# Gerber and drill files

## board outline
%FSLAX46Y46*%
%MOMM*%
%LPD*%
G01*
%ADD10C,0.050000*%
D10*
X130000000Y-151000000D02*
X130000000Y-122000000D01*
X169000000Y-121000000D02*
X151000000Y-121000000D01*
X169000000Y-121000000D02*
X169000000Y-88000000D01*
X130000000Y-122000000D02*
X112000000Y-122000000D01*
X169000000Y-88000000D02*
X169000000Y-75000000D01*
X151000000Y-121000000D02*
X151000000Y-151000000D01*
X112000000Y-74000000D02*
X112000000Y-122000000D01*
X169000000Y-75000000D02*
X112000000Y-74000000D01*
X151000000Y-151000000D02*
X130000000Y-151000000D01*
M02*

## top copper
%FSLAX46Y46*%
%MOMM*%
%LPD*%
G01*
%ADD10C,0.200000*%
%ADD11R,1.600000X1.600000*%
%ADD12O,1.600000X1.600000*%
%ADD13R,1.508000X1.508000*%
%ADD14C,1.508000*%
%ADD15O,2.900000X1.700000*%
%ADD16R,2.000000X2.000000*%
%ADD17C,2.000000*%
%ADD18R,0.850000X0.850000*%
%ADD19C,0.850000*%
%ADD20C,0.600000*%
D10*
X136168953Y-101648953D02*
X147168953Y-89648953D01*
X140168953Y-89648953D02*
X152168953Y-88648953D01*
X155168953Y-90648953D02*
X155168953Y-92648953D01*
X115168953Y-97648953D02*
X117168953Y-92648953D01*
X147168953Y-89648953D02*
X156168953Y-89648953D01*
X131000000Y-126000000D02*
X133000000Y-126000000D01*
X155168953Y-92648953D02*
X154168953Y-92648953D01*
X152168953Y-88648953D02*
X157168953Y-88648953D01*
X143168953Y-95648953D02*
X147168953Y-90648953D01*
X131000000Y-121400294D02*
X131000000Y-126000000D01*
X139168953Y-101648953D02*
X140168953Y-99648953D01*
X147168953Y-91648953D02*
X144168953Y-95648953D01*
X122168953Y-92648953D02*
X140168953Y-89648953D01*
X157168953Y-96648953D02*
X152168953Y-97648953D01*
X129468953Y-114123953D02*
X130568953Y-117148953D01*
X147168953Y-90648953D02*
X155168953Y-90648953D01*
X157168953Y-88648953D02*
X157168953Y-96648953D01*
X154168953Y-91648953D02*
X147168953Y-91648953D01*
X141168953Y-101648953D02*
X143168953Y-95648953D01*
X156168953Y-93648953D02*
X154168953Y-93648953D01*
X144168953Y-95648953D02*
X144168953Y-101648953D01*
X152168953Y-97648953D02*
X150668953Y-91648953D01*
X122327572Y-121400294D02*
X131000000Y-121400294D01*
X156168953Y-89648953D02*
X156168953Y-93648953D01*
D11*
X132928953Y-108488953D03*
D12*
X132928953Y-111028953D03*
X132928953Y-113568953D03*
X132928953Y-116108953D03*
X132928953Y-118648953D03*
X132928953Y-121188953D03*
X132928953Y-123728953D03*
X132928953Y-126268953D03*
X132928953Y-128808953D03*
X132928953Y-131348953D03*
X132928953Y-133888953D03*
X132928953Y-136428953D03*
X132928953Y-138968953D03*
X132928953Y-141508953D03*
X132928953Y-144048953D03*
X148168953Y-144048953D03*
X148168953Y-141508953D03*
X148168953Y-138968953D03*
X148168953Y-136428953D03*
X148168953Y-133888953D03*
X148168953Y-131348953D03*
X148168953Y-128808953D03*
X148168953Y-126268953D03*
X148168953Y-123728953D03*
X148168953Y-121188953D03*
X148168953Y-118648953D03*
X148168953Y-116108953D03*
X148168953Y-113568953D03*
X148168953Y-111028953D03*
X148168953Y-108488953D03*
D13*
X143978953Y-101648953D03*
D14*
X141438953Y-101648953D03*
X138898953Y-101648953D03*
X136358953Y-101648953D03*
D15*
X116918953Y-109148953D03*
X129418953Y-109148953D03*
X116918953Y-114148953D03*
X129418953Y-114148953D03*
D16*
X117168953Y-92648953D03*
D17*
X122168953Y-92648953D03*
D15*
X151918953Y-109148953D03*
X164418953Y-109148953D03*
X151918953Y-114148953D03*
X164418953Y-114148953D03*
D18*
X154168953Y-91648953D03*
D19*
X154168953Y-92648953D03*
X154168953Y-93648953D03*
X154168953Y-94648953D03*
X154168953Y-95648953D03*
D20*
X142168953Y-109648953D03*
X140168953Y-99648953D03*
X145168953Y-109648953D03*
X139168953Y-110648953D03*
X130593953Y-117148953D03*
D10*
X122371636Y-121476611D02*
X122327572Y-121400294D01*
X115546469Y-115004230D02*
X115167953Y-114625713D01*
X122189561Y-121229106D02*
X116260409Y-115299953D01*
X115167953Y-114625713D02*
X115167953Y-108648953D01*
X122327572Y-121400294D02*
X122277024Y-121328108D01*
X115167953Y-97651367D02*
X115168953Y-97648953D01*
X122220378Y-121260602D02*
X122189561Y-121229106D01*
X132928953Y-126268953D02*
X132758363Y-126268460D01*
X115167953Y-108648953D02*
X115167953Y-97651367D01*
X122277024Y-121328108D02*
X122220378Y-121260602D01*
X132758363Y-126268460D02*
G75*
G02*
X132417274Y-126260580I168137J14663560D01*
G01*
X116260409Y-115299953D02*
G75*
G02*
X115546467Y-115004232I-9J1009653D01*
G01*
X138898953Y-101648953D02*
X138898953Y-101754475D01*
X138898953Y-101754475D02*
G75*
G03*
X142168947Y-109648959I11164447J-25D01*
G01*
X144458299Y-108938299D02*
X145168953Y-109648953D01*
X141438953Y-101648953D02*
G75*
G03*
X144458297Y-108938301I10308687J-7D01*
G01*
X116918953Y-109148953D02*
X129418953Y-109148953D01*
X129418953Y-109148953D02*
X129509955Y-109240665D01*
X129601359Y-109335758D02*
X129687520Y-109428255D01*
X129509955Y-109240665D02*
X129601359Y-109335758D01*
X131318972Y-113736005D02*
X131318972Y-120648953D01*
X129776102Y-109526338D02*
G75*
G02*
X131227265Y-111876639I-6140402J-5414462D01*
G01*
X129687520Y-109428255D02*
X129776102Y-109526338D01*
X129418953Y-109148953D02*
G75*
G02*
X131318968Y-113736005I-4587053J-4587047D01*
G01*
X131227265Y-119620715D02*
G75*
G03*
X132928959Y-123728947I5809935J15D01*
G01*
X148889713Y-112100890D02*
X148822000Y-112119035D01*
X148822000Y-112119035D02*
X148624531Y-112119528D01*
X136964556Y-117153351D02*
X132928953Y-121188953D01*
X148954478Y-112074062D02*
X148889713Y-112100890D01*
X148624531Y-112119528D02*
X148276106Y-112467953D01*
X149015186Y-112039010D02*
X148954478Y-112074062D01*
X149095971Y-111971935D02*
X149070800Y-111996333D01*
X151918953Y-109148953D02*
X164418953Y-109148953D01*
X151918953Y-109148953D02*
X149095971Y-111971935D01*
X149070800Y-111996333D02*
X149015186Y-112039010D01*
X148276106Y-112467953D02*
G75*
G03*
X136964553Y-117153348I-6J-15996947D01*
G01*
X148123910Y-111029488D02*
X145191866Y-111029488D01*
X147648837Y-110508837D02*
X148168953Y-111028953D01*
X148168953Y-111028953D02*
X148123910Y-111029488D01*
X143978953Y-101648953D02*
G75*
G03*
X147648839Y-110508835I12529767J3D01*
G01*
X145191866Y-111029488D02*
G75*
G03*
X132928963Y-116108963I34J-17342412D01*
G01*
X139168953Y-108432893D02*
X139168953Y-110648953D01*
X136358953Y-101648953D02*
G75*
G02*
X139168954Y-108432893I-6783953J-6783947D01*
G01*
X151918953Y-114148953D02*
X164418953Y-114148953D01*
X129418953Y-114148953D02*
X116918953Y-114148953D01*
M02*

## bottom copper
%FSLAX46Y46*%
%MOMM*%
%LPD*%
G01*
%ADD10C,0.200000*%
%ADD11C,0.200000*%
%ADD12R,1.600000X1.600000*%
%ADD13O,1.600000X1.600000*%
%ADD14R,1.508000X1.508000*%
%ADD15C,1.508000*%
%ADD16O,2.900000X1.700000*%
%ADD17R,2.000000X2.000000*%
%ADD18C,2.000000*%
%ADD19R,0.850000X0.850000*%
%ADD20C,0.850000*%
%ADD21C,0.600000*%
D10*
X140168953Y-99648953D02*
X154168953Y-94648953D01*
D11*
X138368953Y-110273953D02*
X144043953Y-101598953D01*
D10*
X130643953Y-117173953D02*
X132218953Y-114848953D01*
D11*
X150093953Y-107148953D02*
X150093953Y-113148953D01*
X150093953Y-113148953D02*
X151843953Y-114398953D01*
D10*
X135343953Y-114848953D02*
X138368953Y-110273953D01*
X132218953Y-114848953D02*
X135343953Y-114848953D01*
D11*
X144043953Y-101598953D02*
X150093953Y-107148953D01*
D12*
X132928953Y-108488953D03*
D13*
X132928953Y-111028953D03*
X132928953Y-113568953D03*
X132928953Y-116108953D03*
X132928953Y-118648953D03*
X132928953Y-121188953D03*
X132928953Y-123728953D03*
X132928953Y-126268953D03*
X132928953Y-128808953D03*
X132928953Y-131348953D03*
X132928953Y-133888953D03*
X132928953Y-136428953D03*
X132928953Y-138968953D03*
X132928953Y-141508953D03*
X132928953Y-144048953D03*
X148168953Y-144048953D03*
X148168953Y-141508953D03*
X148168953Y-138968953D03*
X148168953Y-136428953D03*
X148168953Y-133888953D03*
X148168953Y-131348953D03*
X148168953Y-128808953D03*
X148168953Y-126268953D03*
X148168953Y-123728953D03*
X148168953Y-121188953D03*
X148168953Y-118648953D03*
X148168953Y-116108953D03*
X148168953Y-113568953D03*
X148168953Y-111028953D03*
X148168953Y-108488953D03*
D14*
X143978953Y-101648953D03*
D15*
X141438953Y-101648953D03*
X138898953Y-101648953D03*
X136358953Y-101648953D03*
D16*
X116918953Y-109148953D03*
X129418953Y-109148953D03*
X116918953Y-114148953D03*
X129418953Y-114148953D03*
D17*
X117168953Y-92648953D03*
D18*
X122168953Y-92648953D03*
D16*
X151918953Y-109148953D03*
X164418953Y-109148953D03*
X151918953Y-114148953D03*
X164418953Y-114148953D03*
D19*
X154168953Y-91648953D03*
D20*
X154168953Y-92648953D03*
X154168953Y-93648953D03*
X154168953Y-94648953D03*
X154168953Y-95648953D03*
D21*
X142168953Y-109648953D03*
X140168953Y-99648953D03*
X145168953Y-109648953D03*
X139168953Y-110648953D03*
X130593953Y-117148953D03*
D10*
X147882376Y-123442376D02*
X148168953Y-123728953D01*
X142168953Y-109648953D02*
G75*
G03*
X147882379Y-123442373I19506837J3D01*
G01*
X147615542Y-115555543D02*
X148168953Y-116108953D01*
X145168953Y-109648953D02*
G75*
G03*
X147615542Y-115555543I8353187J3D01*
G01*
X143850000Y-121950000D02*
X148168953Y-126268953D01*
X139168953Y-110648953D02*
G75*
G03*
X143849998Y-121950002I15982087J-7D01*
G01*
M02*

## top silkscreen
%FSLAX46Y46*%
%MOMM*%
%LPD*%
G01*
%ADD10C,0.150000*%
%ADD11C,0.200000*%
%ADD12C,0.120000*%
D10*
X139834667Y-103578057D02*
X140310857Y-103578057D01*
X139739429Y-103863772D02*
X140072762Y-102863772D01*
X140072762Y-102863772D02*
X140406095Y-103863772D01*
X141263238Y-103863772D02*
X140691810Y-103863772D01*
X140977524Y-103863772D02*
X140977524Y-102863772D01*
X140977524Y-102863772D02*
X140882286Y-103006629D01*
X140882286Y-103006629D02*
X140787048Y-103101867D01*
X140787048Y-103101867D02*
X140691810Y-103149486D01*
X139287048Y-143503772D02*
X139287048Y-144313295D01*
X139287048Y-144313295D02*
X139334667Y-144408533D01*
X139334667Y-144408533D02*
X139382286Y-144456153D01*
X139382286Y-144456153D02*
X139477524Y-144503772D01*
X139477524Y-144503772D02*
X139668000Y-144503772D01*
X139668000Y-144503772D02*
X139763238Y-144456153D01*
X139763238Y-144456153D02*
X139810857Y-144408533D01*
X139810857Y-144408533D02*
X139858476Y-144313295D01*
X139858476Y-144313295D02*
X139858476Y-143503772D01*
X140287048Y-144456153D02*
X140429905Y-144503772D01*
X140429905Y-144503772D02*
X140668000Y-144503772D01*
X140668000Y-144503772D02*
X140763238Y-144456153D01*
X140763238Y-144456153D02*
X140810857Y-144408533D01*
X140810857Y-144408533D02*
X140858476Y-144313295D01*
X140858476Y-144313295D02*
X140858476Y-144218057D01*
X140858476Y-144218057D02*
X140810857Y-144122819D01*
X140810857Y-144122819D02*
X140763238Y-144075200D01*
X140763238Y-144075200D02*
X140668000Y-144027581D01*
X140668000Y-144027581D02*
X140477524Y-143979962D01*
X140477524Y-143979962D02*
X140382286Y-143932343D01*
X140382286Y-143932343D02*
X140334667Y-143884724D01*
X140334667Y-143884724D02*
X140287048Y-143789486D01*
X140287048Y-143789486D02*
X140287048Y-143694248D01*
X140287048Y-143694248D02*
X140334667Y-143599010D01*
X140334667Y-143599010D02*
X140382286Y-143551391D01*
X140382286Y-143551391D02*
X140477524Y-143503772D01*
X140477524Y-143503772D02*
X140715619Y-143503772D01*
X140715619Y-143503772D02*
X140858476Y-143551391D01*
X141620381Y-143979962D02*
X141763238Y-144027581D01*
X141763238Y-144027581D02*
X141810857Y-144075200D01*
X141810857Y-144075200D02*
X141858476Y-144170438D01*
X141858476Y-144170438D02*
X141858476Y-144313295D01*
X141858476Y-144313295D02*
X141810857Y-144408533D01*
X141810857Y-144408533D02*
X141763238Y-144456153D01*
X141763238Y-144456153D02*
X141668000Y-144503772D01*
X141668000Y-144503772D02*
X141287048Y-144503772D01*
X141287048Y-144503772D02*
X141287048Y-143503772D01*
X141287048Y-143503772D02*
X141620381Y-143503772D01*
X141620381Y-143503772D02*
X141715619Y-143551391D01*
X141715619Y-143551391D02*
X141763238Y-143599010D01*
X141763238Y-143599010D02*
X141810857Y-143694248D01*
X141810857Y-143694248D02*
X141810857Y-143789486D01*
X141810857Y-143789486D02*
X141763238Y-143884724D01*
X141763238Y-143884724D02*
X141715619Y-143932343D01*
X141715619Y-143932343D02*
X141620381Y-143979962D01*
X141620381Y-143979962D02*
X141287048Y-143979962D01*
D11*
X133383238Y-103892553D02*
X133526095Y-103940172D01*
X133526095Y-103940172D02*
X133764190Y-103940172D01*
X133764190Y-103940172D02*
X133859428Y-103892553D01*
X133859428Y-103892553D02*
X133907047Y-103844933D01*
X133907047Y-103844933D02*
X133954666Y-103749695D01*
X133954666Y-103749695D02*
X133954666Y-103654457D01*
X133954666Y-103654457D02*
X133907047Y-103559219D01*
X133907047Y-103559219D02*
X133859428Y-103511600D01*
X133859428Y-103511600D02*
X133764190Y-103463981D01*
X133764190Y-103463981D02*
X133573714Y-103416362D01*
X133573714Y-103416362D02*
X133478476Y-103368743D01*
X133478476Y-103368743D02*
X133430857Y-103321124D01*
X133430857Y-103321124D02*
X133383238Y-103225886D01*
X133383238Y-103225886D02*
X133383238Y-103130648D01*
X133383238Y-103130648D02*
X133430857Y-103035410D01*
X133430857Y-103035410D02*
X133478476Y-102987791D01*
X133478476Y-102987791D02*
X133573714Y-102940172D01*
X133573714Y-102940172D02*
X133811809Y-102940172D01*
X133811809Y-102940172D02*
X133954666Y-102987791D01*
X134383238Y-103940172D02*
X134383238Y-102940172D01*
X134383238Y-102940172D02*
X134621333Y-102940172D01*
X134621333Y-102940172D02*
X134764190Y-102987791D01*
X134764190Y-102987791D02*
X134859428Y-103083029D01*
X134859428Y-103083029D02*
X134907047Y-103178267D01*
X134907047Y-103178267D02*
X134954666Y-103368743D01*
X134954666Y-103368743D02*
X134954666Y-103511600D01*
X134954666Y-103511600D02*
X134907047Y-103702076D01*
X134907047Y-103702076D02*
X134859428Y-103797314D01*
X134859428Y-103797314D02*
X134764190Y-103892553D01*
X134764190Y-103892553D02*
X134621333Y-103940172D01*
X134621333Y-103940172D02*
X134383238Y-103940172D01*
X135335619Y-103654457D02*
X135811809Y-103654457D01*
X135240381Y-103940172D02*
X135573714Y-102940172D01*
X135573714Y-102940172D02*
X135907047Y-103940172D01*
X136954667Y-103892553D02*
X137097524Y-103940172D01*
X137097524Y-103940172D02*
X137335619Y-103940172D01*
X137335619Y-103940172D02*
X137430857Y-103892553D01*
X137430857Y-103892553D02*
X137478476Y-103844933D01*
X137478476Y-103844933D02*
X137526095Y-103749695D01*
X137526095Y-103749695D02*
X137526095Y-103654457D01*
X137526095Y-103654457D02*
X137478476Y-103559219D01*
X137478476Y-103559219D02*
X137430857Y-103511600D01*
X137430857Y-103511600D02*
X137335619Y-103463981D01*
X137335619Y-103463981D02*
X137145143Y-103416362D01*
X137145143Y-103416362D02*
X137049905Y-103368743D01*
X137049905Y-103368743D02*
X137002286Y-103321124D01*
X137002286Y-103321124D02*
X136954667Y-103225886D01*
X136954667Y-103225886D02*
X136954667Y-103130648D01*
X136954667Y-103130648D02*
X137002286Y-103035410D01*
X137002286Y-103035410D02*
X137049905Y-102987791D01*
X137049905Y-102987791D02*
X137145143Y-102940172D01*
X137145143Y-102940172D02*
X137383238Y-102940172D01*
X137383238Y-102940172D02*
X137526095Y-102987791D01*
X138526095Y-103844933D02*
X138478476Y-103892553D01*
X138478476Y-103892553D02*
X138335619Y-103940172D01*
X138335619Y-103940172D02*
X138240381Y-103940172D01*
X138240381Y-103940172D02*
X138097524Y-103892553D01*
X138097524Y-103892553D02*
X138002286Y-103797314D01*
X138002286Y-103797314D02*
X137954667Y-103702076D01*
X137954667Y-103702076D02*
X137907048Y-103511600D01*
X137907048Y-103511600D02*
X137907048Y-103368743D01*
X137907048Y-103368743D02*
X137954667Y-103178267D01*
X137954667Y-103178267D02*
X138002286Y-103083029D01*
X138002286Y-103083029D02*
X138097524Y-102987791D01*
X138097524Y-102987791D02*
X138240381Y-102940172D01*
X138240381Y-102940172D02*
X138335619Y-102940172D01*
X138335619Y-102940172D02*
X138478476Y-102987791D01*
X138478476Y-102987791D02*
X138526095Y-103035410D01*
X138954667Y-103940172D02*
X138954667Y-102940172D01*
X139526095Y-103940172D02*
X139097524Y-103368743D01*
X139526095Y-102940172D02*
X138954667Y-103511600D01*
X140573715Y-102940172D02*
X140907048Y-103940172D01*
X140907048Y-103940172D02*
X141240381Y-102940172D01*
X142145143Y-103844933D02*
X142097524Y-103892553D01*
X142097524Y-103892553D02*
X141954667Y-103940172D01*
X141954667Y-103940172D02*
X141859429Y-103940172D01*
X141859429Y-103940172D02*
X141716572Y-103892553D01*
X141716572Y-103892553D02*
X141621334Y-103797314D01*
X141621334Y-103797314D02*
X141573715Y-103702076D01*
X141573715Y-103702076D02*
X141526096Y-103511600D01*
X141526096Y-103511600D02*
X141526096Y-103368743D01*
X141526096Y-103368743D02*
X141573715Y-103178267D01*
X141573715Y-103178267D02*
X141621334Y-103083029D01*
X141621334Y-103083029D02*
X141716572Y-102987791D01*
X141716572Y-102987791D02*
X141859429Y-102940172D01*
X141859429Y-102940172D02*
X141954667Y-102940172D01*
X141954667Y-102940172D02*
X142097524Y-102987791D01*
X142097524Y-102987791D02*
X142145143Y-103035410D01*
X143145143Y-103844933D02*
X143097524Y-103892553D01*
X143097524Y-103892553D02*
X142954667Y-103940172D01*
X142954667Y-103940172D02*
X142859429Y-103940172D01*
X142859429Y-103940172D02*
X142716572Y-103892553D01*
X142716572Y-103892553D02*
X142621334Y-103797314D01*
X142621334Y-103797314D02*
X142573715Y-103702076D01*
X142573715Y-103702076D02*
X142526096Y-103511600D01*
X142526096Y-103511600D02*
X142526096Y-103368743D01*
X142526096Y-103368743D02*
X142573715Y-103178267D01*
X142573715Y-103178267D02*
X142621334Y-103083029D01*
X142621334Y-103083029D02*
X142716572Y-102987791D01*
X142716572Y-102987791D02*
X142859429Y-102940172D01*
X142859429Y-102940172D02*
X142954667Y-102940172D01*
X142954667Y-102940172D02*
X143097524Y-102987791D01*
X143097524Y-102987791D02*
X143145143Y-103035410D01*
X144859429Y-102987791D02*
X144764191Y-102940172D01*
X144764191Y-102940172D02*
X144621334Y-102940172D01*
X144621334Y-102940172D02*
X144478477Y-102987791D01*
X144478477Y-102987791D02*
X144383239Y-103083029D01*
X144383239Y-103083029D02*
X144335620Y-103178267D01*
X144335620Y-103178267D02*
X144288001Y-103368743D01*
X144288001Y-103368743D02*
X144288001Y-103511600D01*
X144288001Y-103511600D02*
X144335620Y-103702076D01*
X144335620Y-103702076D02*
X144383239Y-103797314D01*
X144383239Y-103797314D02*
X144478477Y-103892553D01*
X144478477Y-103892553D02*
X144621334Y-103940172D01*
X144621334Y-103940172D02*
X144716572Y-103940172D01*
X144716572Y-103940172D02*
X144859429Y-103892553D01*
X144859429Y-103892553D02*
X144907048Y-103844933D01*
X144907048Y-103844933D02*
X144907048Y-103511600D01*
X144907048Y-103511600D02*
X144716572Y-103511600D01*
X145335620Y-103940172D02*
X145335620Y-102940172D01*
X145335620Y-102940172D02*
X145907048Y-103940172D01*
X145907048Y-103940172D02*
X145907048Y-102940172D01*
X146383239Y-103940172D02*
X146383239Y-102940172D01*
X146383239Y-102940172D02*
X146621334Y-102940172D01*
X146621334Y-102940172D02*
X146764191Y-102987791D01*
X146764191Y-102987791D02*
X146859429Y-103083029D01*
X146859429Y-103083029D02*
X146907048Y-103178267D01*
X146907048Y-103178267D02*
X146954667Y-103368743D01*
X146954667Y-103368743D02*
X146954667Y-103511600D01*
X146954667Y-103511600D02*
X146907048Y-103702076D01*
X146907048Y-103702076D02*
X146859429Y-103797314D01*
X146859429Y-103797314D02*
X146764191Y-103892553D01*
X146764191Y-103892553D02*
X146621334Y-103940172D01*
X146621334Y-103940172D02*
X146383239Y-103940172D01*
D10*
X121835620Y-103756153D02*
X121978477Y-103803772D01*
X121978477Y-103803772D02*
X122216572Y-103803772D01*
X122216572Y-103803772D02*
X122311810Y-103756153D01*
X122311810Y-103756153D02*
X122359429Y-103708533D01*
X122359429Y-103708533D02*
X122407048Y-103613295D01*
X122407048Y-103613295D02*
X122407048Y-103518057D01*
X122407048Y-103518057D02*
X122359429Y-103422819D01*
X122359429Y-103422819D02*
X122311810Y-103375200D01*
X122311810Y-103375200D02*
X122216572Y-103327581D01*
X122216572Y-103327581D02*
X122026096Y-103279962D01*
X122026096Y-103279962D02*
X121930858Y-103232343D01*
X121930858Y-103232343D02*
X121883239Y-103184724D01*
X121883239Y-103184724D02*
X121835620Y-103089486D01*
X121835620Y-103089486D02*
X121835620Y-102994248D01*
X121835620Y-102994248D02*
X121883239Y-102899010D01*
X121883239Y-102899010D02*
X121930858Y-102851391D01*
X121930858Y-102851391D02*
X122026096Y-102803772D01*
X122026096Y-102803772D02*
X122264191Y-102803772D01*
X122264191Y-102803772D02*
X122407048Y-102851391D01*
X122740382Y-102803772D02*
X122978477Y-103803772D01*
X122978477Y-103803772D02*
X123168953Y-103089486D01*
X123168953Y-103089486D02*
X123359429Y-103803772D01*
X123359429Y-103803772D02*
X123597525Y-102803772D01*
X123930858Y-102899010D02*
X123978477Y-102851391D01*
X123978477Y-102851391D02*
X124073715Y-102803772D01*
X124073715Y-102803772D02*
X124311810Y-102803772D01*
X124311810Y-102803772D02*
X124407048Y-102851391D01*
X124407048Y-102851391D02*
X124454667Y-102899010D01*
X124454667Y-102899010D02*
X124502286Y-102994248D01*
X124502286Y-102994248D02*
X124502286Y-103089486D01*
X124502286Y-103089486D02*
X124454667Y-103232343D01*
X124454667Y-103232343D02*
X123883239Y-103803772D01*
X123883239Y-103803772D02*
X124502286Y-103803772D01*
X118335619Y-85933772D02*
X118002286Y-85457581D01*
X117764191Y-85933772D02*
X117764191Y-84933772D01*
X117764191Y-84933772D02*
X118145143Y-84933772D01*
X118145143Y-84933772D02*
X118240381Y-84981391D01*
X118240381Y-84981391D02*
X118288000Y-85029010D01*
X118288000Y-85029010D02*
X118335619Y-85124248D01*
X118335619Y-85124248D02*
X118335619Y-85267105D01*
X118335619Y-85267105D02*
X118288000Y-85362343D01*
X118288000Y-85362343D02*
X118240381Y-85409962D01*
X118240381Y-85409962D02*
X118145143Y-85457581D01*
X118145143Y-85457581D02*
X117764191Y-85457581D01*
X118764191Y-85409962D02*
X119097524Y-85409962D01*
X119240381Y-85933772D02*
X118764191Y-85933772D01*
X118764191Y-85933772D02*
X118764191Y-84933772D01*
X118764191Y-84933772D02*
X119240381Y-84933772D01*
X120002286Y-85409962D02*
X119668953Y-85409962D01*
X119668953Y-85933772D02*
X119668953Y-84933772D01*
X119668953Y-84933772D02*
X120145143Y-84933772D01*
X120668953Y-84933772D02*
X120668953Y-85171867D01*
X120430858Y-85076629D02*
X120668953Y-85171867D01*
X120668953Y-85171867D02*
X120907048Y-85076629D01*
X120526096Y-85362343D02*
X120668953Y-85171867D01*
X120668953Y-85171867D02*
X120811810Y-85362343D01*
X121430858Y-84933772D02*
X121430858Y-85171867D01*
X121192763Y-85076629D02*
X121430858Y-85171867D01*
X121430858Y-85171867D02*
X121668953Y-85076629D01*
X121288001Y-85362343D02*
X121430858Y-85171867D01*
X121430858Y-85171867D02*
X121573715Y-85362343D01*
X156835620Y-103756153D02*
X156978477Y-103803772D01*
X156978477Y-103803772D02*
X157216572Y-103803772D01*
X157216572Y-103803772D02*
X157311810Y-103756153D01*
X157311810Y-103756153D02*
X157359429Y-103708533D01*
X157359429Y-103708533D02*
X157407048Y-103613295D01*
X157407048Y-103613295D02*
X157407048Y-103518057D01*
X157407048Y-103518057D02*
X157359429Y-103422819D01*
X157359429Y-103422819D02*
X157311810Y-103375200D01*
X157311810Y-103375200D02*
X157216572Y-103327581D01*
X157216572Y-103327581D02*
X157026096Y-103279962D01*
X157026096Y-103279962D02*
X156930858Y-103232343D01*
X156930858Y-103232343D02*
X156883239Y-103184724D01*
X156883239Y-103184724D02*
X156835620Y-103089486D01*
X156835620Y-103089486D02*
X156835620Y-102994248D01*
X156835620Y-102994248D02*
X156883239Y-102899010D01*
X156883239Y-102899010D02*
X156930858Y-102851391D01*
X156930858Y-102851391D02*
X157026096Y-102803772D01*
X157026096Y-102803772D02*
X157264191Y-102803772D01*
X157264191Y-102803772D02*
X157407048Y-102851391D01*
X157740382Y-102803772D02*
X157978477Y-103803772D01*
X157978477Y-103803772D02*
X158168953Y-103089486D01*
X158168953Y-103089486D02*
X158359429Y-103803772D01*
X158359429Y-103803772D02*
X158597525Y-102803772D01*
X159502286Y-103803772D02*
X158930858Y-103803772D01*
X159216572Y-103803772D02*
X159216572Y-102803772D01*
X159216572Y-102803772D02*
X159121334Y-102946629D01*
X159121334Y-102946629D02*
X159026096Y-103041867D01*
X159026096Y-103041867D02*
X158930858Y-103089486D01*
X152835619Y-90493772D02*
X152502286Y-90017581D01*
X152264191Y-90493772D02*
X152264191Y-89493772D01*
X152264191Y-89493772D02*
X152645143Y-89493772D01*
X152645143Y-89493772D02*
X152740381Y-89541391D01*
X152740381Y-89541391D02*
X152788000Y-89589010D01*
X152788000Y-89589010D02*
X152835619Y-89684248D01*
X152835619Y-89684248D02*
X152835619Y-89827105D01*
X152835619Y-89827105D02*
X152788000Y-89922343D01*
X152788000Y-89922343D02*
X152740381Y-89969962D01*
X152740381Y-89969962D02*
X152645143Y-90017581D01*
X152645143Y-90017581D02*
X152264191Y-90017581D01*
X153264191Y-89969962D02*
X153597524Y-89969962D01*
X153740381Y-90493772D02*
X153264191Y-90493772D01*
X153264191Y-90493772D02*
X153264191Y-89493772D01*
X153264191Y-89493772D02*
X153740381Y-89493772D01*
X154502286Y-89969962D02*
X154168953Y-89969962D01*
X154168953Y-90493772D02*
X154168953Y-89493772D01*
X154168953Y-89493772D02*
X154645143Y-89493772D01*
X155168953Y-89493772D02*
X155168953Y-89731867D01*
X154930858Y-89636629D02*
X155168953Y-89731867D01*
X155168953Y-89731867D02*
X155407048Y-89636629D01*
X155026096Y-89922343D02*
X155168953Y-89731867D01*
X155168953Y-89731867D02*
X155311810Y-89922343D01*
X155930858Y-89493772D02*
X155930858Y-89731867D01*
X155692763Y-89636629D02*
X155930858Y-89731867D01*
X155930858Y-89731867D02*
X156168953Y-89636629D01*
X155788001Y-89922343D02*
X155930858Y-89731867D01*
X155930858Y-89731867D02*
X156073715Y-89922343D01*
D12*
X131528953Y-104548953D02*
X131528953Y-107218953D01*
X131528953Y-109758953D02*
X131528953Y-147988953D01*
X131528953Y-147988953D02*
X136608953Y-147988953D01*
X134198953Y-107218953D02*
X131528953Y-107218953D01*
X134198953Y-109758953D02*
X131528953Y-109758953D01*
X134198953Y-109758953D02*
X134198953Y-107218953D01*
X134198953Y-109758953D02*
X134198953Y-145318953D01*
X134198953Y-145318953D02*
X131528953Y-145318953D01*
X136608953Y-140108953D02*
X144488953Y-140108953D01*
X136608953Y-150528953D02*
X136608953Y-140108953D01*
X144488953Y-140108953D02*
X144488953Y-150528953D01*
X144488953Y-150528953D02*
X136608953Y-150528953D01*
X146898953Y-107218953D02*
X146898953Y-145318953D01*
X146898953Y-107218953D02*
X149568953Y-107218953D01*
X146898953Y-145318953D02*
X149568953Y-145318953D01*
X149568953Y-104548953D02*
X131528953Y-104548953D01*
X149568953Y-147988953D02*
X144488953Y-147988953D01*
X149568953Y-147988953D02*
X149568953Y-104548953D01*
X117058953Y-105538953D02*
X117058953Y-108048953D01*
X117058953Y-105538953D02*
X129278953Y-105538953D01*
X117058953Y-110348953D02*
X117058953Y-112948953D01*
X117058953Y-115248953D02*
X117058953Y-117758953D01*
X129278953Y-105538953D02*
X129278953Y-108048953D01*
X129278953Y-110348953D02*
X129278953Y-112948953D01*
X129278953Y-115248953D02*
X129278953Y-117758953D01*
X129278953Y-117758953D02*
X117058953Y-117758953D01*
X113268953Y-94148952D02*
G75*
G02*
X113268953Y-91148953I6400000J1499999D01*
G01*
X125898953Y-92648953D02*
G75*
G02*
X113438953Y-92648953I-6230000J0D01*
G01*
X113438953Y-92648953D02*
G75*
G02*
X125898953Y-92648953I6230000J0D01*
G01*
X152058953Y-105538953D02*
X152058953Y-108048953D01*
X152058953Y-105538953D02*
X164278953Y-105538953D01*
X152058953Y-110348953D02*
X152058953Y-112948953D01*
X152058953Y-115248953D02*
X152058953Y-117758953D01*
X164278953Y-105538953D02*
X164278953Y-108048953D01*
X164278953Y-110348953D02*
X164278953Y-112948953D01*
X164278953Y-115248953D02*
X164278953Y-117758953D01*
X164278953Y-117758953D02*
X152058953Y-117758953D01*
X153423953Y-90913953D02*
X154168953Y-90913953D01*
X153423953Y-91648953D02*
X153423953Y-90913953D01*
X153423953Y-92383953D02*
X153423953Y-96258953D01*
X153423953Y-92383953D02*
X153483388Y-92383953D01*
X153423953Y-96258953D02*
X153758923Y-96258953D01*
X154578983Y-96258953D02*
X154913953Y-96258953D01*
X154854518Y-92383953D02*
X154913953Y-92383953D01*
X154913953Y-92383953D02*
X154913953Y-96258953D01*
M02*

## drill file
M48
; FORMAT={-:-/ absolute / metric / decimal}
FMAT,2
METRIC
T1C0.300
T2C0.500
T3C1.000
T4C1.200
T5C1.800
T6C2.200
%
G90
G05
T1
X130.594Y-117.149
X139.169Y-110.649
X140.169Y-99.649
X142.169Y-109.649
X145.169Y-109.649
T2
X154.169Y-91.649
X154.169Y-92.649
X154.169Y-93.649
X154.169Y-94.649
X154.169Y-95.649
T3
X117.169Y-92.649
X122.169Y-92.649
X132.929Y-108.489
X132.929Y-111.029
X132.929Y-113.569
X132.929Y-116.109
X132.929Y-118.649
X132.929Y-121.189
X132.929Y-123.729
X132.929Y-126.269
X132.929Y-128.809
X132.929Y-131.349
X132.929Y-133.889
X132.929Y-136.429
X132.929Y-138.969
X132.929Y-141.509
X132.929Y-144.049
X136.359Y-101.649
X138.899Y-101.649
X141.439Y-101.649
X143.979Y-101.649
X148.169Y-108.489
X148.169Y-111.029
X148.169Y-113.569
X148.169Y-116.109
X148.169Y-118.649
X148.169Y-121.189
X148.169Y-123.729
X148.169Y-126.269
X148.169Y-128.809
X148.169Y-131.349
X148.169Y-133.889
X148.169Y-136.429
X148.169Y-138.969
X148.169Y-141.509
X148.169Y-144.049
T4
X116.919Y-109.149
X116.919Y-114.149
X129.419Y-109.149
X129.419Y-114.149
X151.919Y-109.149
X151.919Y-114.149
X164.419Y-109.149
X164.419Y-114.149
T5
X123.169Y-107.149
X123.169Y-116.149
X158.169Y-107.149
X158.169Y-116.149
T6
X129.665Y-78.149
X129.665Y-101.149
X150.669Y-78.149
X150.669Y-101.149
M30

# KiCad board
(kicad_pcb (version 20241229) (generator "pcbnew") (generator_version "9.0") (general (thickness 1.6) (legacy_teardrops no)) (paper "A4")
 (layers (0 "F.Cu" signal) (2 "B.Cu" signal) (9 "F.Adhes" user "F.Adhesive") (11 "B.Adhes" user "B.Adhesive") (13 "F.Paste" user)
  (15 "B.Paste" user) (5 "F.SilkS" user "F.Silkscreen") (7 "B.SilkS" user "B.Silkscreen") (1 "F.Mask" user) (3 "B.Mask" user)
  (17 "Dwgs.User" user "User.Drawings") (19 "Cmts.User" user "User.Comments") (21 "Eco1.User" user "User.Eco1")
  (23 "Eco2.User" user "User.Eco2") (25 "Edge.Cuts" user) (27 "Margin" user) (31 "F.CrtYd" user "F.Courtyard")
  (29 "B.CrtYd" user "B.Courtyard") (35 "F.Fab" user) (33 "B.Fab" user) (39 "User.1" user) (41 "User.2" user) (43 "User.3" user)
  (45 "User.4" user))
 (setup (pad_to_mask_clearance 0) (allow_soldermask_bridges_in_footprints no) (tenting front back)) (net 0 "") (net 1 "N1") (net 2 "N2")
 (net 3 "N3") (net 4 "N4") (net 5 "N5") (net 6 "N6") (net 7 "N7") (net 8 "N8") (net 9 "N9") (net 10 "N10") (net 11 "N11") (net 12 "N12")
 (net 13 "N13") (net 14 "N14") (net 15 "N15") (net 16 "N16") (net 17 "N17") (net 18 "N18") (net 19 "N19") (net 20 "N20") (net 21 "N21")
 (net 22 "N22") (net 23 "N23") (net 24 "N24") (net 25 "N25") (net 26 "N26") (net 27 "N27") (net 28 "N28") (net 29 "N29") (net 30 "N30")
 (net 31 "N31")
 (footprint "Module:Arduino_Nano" (layer "F.Cu") (at 132.928953 108.488953)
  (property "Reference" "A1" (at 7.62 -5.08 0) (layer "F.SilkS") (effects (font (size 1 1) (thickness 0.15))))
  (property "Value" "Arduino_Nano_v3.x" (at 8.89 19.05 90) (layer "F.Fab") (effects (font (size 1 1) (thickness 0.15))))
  (fp_line (start -1.4 -3.94) (end -1.4 -1.27) (stroke (width 0.12) (type solid)) (layer "F.SilkS"))
  (fp_line (start -1.4 1.27) (end -1.4 39.5) (stroke (width 0.12) (type solid)) (layer "F.SilkS"))
  (fp_line (start -1.4 39.5) (end 3.68 39.5) (stroke (width 0.12) (type solid)) (layer "F.SilkS"))
  (fp_line (start 1.27 -1.27) (end -1.4 -1.27) (stroke (width 0.12) (type solid)) (layer "F.SilkS"))
  (fp_line (start 1.27 1.27) (end -1.4 1.27) (stroke (width 0.12) (type solid)) (layer "F.SilkS"))
  (fp_line (start 1.27 1.27) (end 1.27 -1.27) (stroke (width 0.12) (type solid)) (layer "F.SilkS"))
  (fp_line (start 1.27 1.27) (end 1.27 36.83) (stroke (width 0.12) (type solid)) (layer "F.SilkS"))
  (fp_line (start 1.27 36.83) (end -1.4 36.83) (stroke (width 0.12) (type solid)) (layer "F.SilkS"))
  (fp_line (start 3.68 31.62) (end 11.56 31.62) (stroke (width 0.12) (type solid)) (layer "F.SilkS"))
  (fp_line (start 3.68 42.04) (end 3.68 31.62) (stroke (width 0.12) (type solid)) (layer "F.SilkS"))
  (fp_line (start 11.56 31.62) (end 11.56 42.04) (stroke (width 0.12) (type solid)) (layer "F.SilkS"))
  (fp_line (start 11.56 42.04) (end 3.68 42.04) (stroke (width 0.12) (type solid)) (layer "F.SilkS"))
  (fp_line (start 13.97 -1.27) (end 13.97 36.83) (stroke (width 0.12) (type solid)) (layer "F.SilkS"))
  (fp_line (start 13.97 -1.27) (end 16.64 -1.27) (stroke (width 0.12) (type solid)) (layer "F.SilkS"))
  (fp_line (start 13.97 36.83) (end 16.64 36.83) (stroke (width 0.12) (type solid)) (layer "F.SilkS"))
  (fp_line (start 16.64 -3.94) (end -1.4 -3.94) (stroke (width 0.12) (type solid)) (layer "F.SilkS"))
  (fp_line (start 16.64 39.5) (end 11.56 39.5) (stroke (width 0.12) (type solid)) (layer "F.SilkS"))
  (fp_line (start 16.64 39.5) (end 16.64 -3.94) (stroke (width 0.12) (type solid)) (layer "F.SilkS"))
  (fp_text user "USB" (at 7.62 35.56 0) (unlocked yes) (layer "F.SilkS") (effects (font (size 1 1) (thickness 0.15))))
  (pad "1" thru_hole rect (at 0 0) (size 1.6 1.6) (drill 1) (layers "*.Cu" "*.Mask") (remove_unused_layers no) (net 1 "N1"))
  (pad "2" thru_hole oval (at 0 2.54) (size 1.6 1.6) (drill 1) (layers "*.Cu" "*.Mask") (remove_unused_layers no) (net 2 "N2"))
  (pad "3" thru_hole oval (at 0 5.08) (size 1.6 1.6) (drill 1) (layers "*.Cu" "*.Mask") (remove_unused_layers no) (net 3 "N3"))
  (pad "4" thru_hole oval (at 0 7.62) (size 1.6 1.6) (drill 1) (layers "*.Cu" "*.Mask") (remove_unused_layers no) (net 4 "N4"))
  (pad "5" thru_hole oval (at 0 10.16) (size 1.6 1.6) (drill 1) (layers "*.Cu" "*.Mask") (remove_unused_layers no) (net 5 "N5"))
  (pad "6" thru_hole oval (at 0 12.7) (size 1.6 1.6) (drill 1) (layers "*.Cu" "*.Mask") (remove_unused_layers no) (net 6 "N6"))
  (pad "7" thru_hole oval (at 0 15.24) (size 1.6 1.6) (drill 1) (layers "*.Cu" "*.Mask") (remove_unused_layers no) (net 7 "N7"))
  (pad "8" thru_hole oval (at 0 17.78) (size 1.6 1.6) (drill 1) (layers "*.Cu" "*.Mask") (remove_unused_layers no) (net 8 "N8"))
  (pad "9" thru_hole oval (at 0 20.32) (size 1.6 1.6) (drill 1) (layers "*.Cu" "*.Mask") (remove_unused_layers no) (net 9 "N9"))
  (pad "10" thru_hole oval (at 0 22.86) (size 1.6 1.6) (drill 1) (layers "*.Cu" "*.Mask") (remove_unused_layers no) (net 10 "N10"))
  (pad "11" thru_hole oval (at 0 25.4) (size 1.6 1.6) (drill 1) (layers "*.Cu" "*.Mask") (remove_unused_layers no) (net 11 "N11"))
  (pad "12" thru_hole oval (at 0 27.94) (size 1.6 1.6) (drill 1) (layers "*.Cu" "*.Mask") (remove_unused_layers no) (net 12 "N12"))
  (pad "13" thru_hole oval (at 0 30.48) (size 1.6 1.6) (drill 1) (layers "*.Cu" "*.Mask") (remove_unused_layers no) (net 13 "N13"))
  (pad "14" thru_hole oval (at 0 33.02) (size 1.6 1.6) (drill 1) (layers "*.Cu" "*.Mask") (remove_unused_layers no) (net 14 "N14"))
  (pad "15" thru_hole oval (at 0 35.56) (size 1.6 1.6) (drill 1) (layers "*.Cu" "*.Mask") (remove_unused_layers no) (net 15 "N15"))
  (pad "16" thru_hole oval (at 15.24 35.56) (size 1.6 1.6) (drill 1) (layers "*.Cu" "*.Mask") (remove_unused_layers no) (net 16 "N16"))
  (pad "17" thru_hole oval (at 15.24 33.02) (size 1.6 1.6) (drill 1) (layers "*.Cu" "*.Mask") (remove_unused_layers no) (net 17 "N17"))
  (pad "18" thru_hole oval (at 15.24 30.48) (size 1.6 1.6) (drill 1) (layers "*.Cu" "*.Mask") (remove_unused_layers no) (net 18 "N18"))
  (pad "19" thru_hole oval (at 15.24 27.94) (size 1.6 1.6) (drill 1) (layers "*.Cu" "*.Mask") (remove_unused_layers no) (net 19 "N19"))
  (pad "20" thru_hole oval (at 15.24 25.4) (size 1.6 1.6) (drill 1) (layers "*.Cu" "*.Mask") (remove_unused_layers no) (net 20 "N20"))
  (pad "21" thru_hole oval (at 15.24 22.86) (size 1.6 1.6) (drill 1) (layers "*.Cu" "*.Mask") (remove_unused_layers no) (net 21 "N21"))
  (pad "22" thru_hole oval (at 15.24 20.32) (size 1.6 1.6) (drill 1) (layers "*.Cu" "*.Mask") (remove_unused_layers no) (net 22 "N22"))
  (pad "23" thru_hole oval (at 15.24 17.78) (size 1.6 1.6) (drill 1) (layers "*.Cu" "*.Mask") (remove_unused_layers no) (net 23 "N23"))
  (pad "24" thru_hole oval (at 15.24 15.24) (size 1.6 1.6) (drill 1) (layers "*.Cu" "*.Mask") (remove_unused_layers no) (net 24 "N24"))
  (pad "25" thru_hole oval (at 15.24 12.7) (size 1.6 1.6) (drill 1) (layers "*.Cu" "*.Mask") (remove_unused_layers no) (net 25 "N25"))
  (pad "26" thru_hole oval (at 15.24 10.16) (size 1.6 1.6) (drill 1) (layers "*.Cu" "*.Mask") (remove_unused_layers no) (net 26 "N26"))
  (pad "27" thru_hole oval (at 15.24 7.62) (size 1.6 1.6) (drill 1) (layers "*.Cu" "*.Mask") (remove_unused_layers no) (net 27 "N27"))
  (pad "28" thru_hole oval (at 15.24 5.08) (size 1.6 1.6) (drill 1) (layers "*.Cu" "*.Mask") (remove_unused_layers no) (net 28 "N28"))
  (pad "29" thru_hole oval (at 15.24 2.54) (size 1.6 1.6) (drill 1) (layers "*.Cu" "*.Mask") (remove_unused_layers no) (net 4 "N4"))
  (pad "30" thru_hole oval (at 15.24 0) (size 1.6 1.6) (drill 1) (layers "*.Cu" "*.Mask") (remove_unused_layers no) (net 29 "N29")))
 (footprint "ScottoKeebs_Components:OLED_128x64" (layer "F.Cu") (at 140.168953 89.648953)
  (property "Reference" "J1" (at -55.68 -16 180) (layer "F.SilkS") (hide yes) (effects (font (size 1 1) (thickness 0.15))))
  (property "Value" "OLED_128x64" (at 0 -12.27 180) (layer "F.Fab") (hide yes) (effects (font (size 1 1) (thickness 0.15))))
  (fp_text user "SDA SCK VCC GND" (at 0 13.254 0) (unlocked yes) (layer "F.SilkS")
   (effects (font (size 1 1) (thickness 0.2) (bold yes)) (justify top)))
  (pad "" np_thru_hole circle (at -10.50445 -11.5 180) (size 2.2 2.2) (drill 2.2) (layers "*.Cu" "*.Mask") (solder_mask_margin 0.102))
  (pad "" np_thru_hole circle (at -10.50445 11.5 180) (size 2.2 2.2) (drill 2.2) (layers "*.Cu" "*.Mask") (solder_mask_margin 0.102))
  (pad "" np_thru_hole circle (at 10.5 -11.5 180) (size 2.2 2.2) (drill 2.2) (layers "*.Cu" "*.Mask") (solder_mask_margin 0.102))
  (pad "" np_thru_hole circle (at 10.5 11.5 180) (size 2.2 2.2) (drill 2.2) (layers "*.Cu" "*.Mask") (solder_mask_margin 0.102))
  (pad "1" thru_hole rect (at 3.81 12 180) (size 1.508 1.508) (drill 1) (layers "*.Cu" "*.Mask") (remove_unused_layers no) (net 4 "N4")
   (solder_mask_margin 0.102))
  (pad "2" thru_hole circle (at 1.27 12 180) (size 1.508 1.508) (drill 1) (layers "*.Cu" "*.Mask") (remove_unused_layers no) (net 27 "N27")
   (solder_mask_margin 0.102))
  (pad "3" thru_hole circle (at -1.27 12 180) (size 1.508 1.508) (drill 1) (layers "*.Cu" "*.Mask") (remove_unused_layers no) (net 24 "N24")
   (solder_mask_margin 0.102))
  (pad "4" thru_hole circle (at -3.81 12 180) (size 1.508 1.508) (drill 1) (layers "*.Cu" "*.Mask") (remove_unused_layers no) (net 23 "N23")
   (solder_mask_margin 0.102)))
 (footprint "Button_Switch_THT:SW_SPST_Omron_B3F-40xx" (layer "F.Cu") (at 116.918953 109.148953)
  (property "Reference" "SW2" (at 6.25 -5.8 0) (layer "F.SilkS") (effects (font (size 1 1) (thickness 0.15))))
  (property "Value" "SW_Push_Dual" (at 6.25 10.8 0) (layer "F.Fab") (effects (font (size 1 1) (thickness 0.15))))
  (fp_line (start 0.14 -3.61) (end 0.14 -1.1) (stroke (width 0.12) (type default)) (layer "F.SilkS"))
  (fp_line (start 0.14 -3.61) (end 12.36 -3.61) (stroke (width 0.12) (type default)) (layer "F.SilkS"))
  (fp_line (start 0.14 1.2) (end 0.14 3.8) (stroke (width 0.12) (type default)) (layer "F.SilkS"))
  (fp_line (start 0.14 6.1) (end 0.14 8.61) (stroke (width 0.12) (type default)) (layer "F.SilkS"))
  (fp_line (start 12.36 -3.61) (end 12.36 -1.1) (stroke (width 0.12) (type default)) (layer "F.SilkS"))
  (fp_line (start 12.36 1.2) (end 12.36 3.8) (stroke (width 0.12) (type default)) (layer "F.SilkS"))
  (fp_line (start 12.36 6.1) (end 12.36 8.61) (stroke (width 0.12) (type default)) (layer "F.SilkS"))
  (fp_line (start 12.36 8.61) (end 0.14 8.61) (stroke (width 0.12) (type default)) (layer "F.SilkS"))
  (pad "" np_thru_hole circle (at 6.25 -2) (size 1.8 1.8) (drill 1.8) (layers "*.Cu" "*.Mask"))
  (pad "" np_thru_hole circle (at 6.25 7) (size 1.8 1.8) (drill 1.8) (layers "*.Cu" "*.Mask"))
  (pad "1" thru_hole oval (at 0 0) (size 2.9 1.7) (drill 1.2) (layers "*.Cu" "*.Mask") (remove_unused_layers no) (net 7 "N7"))
  (pad "1" thru_hole oval (at 12.5 0) (size 2.9 1.7) (drill 1.2) (layers "*.Cu" "*.Mask") (remove_unused_layers no) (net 7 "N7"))
  (pad "2" thru_hole oval (at 0 5) (size 2.9 1.7) (drill 1.2) (layers "*.Cu" "*.Mask") (remove_unused_layers no) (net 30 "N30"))
  (pad "2" thru_hole oval (at 12.5 5) (size 2.9 1.7) (drill 1.2) (layers "*.Cu" "*.Mask") (remove_unused_layers no) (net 30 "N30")))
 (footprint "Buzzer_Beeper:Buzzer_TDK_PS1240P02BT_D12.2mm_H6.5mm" (layer "F.Cu") (at 117.168953 92.648953)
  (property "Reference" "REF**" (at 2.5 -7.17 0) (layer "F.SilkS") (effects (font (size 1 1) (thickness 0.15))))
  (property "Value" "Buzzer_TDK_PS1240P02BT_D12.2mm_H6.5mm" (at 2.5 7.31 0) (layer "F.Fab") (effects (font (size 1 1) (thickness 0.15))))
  (fp_arc (start -3.9 1.499999) (mid -4.073431 0) (end -3.9 -1.5) (stroke (width 0.12) (type solid)) (layer "F.SilkS"))
  (fp_circle (center 2.5 0) (end 8.73 0) (stroke (width 0.12) (type solid)) (fill no) (layer "F.SilkS"))
  (pad "1" thru_hole rect (at 0 0) (size 2 2) (drill 1) (layers "*.Cu" "*.Mask") (remove_unused_layers no))
  (pad "2" thru_hole circle (at 5 0) (size 2 2) (drill 1) (layers "*.Cu" "*.Mask") (remove_unused_layers no)))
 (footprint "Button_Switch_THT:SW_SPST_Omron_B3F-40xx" (layer "F.Cu") (at 151.918953 109.148953)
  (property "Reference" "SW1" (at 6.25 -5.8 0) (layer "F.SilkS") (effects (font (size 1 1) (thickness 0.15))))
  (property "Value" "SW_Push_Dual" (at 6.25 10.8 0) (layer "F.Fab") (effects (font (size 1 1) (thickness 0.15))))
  (fp_line (start 0.14 -3.61) (end 0.14 -1.1) (stroke (width 0.12) (type default)) (layer "F.SilkS"))
  (fp_line (start 0.14 -3.61) (end 12.36 -3.61) (stroke (width 0.12) (type default)) (layer "F.SilkS"))
  (fp_line (start 0.14 1.2) (end 0.14 3.8) (stroke (width 0.12) (type default)) (layer "F.SilkS"))
  (fp_line (start 0.14 6.1) (end 0.14 8.61) (stroke (width 0.12) (type default)) (layer "F.SilkS"))
  (fp_line (start 12.36 -3.61) (end 12.36 -1.1) (stroke (width 0.12) (type default)) (layer "F.SilkS"))
  (fp_line (start 12.36 1.2) (end 12.36 3.8) (stroke (width 0.12) (type default)) (layer "F.SilkS"))
  (fp_line (start 12.36 6.1) (end 12.36 8.61) (stroke (width 0.12) (type default)) (layer "F.SilkS"))
  (fp_line (start 12.36 8.61) (end 0.14 8.61) (stroke (width 0.12) (type default)) (layer "F.SilkS"))
  (pad "" np_thru_hole circle (at 6.25 -2) (size 1.8 1.8) (drill 1.8) (layers "*.Cu" "*.Mask"))
  (pad "" np_thru_hole circle (at 6.25 7) (size 1.8 1.8) (drill 1.8) (layers "*.Cu" "*.Mask"))
  (pad "1" thru_hole oval (at 0 0) (size 2.9 1.7) (drill 1.2) (layers "*.Cu" "*.Mask") (remove_unused_layers no) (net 6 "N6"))
  (pad "1" thru_hole oval (at 12.5 0) (size 2.9 1.7) (drill 1.2) (layers "*.Cu" "*.Mask") (remove_unused_layers no) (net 6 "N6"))
  (pad "2" thru_hole oval (at 0 5) (size 2.9 1.7) (drill 1.2) (layers "*.Cu" "*.Mask") (remove_unused_layers no) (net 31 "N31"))
  (pad "2" thru_hole oval (at 12.5 5) (size 2.9 1.7) (drill 1.2) (layers "*.Cu" "*.Mask") (remove_unused_layers no) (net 31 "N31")))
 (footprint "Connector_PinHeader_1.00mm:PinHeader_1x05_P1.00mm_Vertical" (layer "F.Cu") (at 154.168953 91.648953)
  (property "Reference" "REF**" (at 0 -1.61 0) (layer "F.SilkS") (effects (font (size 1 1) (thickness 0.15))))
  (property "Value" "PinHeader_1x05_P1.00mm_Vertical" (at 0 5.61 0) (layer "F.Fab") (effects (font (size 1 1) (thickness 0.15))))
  (fp_line (start -0.745 -0.735) (end 0 -0.735) (stroke (width 0.12) (type solid)) (layer "F.SilkS"))
  (fp_line (start -0.745 0) (end -0.745 -0.735) (stroke (width 0.12) (type solid)) (layer "F.SilkS"))
  (fp_line (start -0.745 0.735) (end -0.745 4.61) (stroke (width 0.12) (type solid)) (layer "F.SilkS"))
  (fp_line (start -0.745 0.735) (end -0.685565 0.735) (stroke (width 0.12) (type solid)) (layer "F.SilkS"))
  (fp_line (start -0.745 4.61) (end -0.41003 4.61) (stroke (width 0.12) (type solid)) (layer "F.SilkS"))
  (fp_line (start 0.41003 4.61) (end 0.745 4.61) (stroke (width 0.12) (type solid)) (layer "F.SilkS"))
  (fp_line (start 0.685565 0.735) (end 0.745 0.735) (stroke (width 0.12) (type solid)) (layer "F.SilkS"))
  (fp_line (start 0.745 0.735) (end 0.745 4.61) (stroke (width 0.12) (type solid)) (layer "F.SilkS"))
  (pad "1" thru_hole rect (at 0 0) (size 0.85 0.85) (drill 0.5) (layers "*.Cu" "*.Mask") (remove_unused_layers no))
  (pad "2" thru_hole circle (at 0 1) (size 0.85 0.85) (drill 0.5) (layers "*.Cu" "*.Mask") (remove_unused_layers no))
  (pad "3" thru_hole circle (at 0 2) (size 0.85 0.85) (drill 0.5) (layers "*.Cu" "*.Mask") (remove_unused_layers no))
  (pad "4" thru_hole circle (at 0 3) (size 0.85 0.85) (drill 0.5) (layers "*.Cu" "*.Mask") (remove_unused_layers no))
  (pad "5" thru_hole circle (at 0 4) (size 0.85 0.85) (drill 0.5) (layers "*.Cu" "*.Mask") (remove_unused_layers no)))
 (gr_line (start 136.168953 101.648953) (end 147.168953 89.648953) (stroke (width 0.2) (type default)) (layer "F.Cu") (net 23))
 (gr_line (start 140.168953 89.648953) (end 152.168953 88.648953) (stroke (width 0.2) (type default)) (layer "F.Cu") (net 4))
 (gr_line (start 155.168953 90.648953) (end 155.168953 92.648953) (stroke (width 0.2) (type default)) (layer "F.Cu") (net 27))
 (gr_line (start 115.168953 97.648953) (end 117.168953 92.648953) (stroke (width 0.2) (type default)) (layer "F.Cu") (net 8))
 (gr_line (start 147.168953 89.648953) (end 156.168953 89.648953) (stroke (width 0.2) (type default)) (layer "F.Cu") (net 23))
 (gr_line (start 131 126) (end 133 126) (stroke (width 0.2) (type default)) (layer "F.Cu") (net 8))
 (gr_line (start 155.168953 92.648953) (end 154.168953 92.648953) (stroke (width 0.2) (type default)) (layer "F.Cu") (net 27))
 (gr_line (start 152.168953 88.648953) (end 157.168953 88.648953) (stroke (width 0.2) (type default)) (layer "F.Cu") (net 4))
 (gr_line (start 143.168953 95.648953) (end 147.168953 90.648953) (stroke (width 0.2) (type default)) (layer "F.Cu") (net 27))
 (gr_line (start 131 121.400294) (end 131 126) (stroke (width 0.2) (type default)) (layer "F.Cu") (net 8))
 (gr_line (start 139.168953 101.648953) (end 140.168953 99.648953) (stroke (width 0.2) (type default)) (layer "F.Cu") (net 24))
 (gr_line (start 147.168953 91.648953) (end 144.168953 95.648953) (stroke (width 0.2) (type default)) (layer "F.Cu") (net 4))
 (gr_line (start 122.168953 92.648953) (end 140.168953 89.648953) (stroke (width 0.2) (type default)) (layer "F.Cu") (net 4))
 (gr_line (start 157.168953 96.648953) (end 152.168953 97.648953) (stroke (width 0.2) (type default)) (layer "F.Cu") (net 4))
 (gr_line (start 129.468953 114.123953) (end 130.568953 117.148953) (stroke (width 0.2) (type default)) (layer "F.Cu") (net 30))
 (gr_line (start 147.168953 90.648953) (end 155.168953 90.648953) (stroke (width 0.2) (type default)) (layer "F.Cu") (net 27))
 (gr_line (start 157.168953 88.648953) (end 157.168953 96.648953) (stroke (width 0.2) (type default)) (layer "F.Cu") (net 4))
 (gr_line (start 154.168953 91.648953) (end 147.168953 91.648953) (stroke (width 0.2) (type default)) (layer "F.Cu") (net 4))
 (gr_line (start 141.168953 101.648953) (end 143.168953 95.648953) (stroke (width 0.2) (type default)) (layer "F.Cu") (net 27))
 (gr_line (start 156.168953 93.648953) (end 154.168953 93.648953) (stroke (width 0.2) (type default)) (layer "F.Cu") (net 23))
 (gr_line (start 144.168953 95.648953) (end 144.168953 101.648953) (stroke (width 0.2) (type default)) (layer "F.Cu") (net 4))
 (gr_line (start 152.168953 97.648953) (end 150.668953 91.648953) (stroke (width 0.2) (type default)) (layer "F.Cu") (net 4))
 (gr_line (start 122.327572 121.400294) (end 131 121.400294) (stroke (width 0.2) (type default)) (layer "F.Cu") (net 8))
 (gr_line (start 156.168953 89.648953) (end 156.168953 93.648953) (stroke (width 0.2) (type default)) (layer "F.Cu") (net 23))
 (gr_line (start 140.168953 99.648953) (end 154.168953 94.648953) (stroke (width 0.2) (type default)) (layer "B.Cu") (net 24))
 (gr_line (start 138.368953 110.273953) (end 144.043953 101.598953) (stroke (width 0.2) (type default)) (layer "B.Cu"))
 (gr_line (start 130.643953 117.173953) (end 132.218953 114.848953) (stroke (width 0.2) (type default)) (layer "B.Cu") (net 30))
 (gr_line (start 150.093953 107.148953) (end 150.093953 113.148953) (stroke (width 0.2) (type default)) (layer "B.Cu"))
 (gr_line (start 150.093953 113.148953) (end 151.843953 114.398953) (stroke (width 0.2) (type default)) (layer "B.Cu"))
 (gr_line (start 135.343953 114.848953) (end 138.368953 110.273953) (stroke (width 0.2) (type default)) (layer "B.Cu") (net 30))
 (gr_line (start 132.218953 114.848953) (end 135.343953 114.848953) (stroke (width 0.2) (type default)) (layer "B.Cu") (net 30))
 (gr_line (start 144.043953 101.598953) (end 150.093953 107.148953) (stroke (width 0.2) (type default)) (layer "B.Cu"))
 (gr_line (start 130 151) (end 130 122) (stroke (width 0.05) (type default)) (layer "Edge.Cuts"))
 (gr_line (start 169 121) (end 151 121) (stroke (width 0.05) (type default)) (layer "Edge.Cuts"))
 (gr_line (start 169 121) (end 169 88) (stroke (width 0.05) (type default)) (layer "Edge.Cuts"))
 (gr_line (start 130 122) (end 112 122) (stroke (width 0.05) (type default)) (layer "Edge.Cuts"))
 (gr_line (start 169 88) (end 169 75) (stroke (width 0.05) (type default)) (layer "Edge.Cuts"))
 (gr_line (start 151 121) (end 151 151) (stroke (width 0.05) (type default)) (layer "Edge.Cuts"))
 (gr_line (start 112 74) (end 112 122) (stroke (width 0.05) (type default)) (layer "Edge.Cuts"))
 (gr_line (start 169 75) (end 112 74) (stroke (width 0.05) (type default)) (layer "Edge.Cuts"))
 (gr_line (start 151 151) (end 130 151) (stroke (width 0.05) (type default)) (layer "Edge.Cuts"))
 (segment (start 122.371636 121.476611) (end 122.327572 121.400294) (width 0.2) (layer "F.Cu") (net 8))
 (segment (start 115.546469 115.00423) (end 115.167953 114.625713) (width 0.2) (layer "F.Cu") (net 8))
 (segment (start 122.189561 121.229106) (end 116.260409 115.299953) (width 0.2) (layer "F.Cu") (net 8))
 (segment (start 115.167953 114.625713) (end 115.167953 108.648953) (width 0.2) (layer "F.Cu") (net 8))
 (segment (start 122.327572 121.400294) (end 122.277024 121.328108) (width 0.2) (layer "F.Cu") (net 8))
 (segment (start 115.167953 97.651367) (end 115.168953 97.648953) (width 0.2) (layer "F.Cu") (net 8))
 (segment (start 122.220378 121.260602) (end 122.189561 121.229106) (width 0.2) (layer "F.Cu") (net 8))
 (segment (start 132.928953 126.268953) (end 132.758363 126.26846) (width 0.2) (layer "F.Cu") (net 8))
 (segment (start 115.167953 108.648953) (end 115.167953 97.651367) (width 0.2) (layer "F.Cu") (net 8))
 (segment (start 122.277024 121.328108) (end 122.220378 121.260602) (width 0.2) (layer "F.Cu") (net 8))
 (arc (start 132.758363 126.26846) (mid 132.587796 126.265512) (end 132.417274 126.26058) (width 0.2) (layer "F.Cu") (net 8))
 (arc (start 116.260409 115.299953) (mid 115.874028 115.223097) (end 115.546469 115.00423) (width 0.2) (layer "F.Cu") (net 8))
 (segment (start 138.898953 101.648953) (end 138.898953 101.754475) (width 0.2) (layer "F.Cu") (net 24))
 (via (at 142.168953 109.648953) (size 0.6) (drill 0.3) (layers "F.Cu" "B.Cu") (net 24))
 (via (at 140.168953 99.648953) (size 0.6) (drill 0.3) (layers "F.Cu" "B.Cu") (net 24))
 (arc (start 138.898953 101.754475) (mid 139.748799 106.026935) (end 142.168953 109.648953) (width 0.2) (layer "F.Cu") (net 24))
 (segment (start 147.882376 123.442376) (end 148.168953 123.728953) (width 0.2) (layer "B.Cu") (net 24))
 (arc (start 142.168953 109.648953) (mid 143.653823 117.1139) (end 147.882376 123.442376) (width 0.2) (layer "B.Cu") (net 24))
 (segment (start 144.458299 108.938299) (end 145.168953 109.648953) (width 0.2) (layer "F.Cu") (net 27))
 (via (at 145.168953 109.648953) (size 0.6) (drill 0.3) (layers "F.Cu" "B.Cu") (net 27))
 (arc (start 141.438953 101.648953) (mid 142.223655 105.593919) (end 144.458299 108.938299) (width 0.2) (layer "F.Cu") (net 27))
 (segment (start 147.615542 115.555543) (end 148.168953 116.108953) (width 0.2) (layer "B.Cu") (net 27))
 (arc (start 145.168953 109.648953) (mid 145.804801 112.845576) (end 147.615542 115.555543) (width 0.2) (layer "B.Cu") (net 27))
 (segment (start 116.918953 109.148953) (end 129.418953 109.148953) (width 0.2) (layer "F.Cu") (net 7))
 (segment (start 129.418953 109.148953) (end 129.509955 109.240665) (width 0.2) (layer "F.Cu") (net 7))
 (segment (start 129.601359 109.335758) (end 129.68752 109.428255) (width 0.2) (layer "F.Cu") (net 7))
 (segment (start 129.509955 109.240665) (end 129.601359 109.335758) (width 0.2) (layer "F.Cu") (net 7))
 (segment (start 131.318972 113.736005) (end 131.318972 120.648953) (width 0.2) (layer "F.Cu") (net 7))
 (arc (start 129.776102 109.526338) (mid 130.601536 110.639862) (end 131.227265 111.876639) (width 0.2) (layer "F.Cu") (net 7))
 (arc (start 129.68752 109.428255) (mid 129.73181 109.477295) (end 129.776102 109.526338) (width 0.2) (layer "F.Cu") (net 7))
 (arc (start 129.418953 109.148953) (mid 130.825173 111.253511) (end 131.318972 113.736005) (width 0.2) (layer "F.Cu") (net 7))
 (arc (start 131.227265 119.620715) (mid 131.66952 121.844077) (end 132.928953 123.728953) (width 0.2) (layer "F.Cu") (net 7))
 (segment (start 148.889713 112.10089) (end 148.822 112.119035) (width 0.2) (layer "F.Cu") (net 6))
 (segment (start 148.822 112.119035) (end 148.624531 112.119528) (width 0.2) (layer "F.Cu") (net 6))
 (segment (start 136.964556 117.153351) (end 132.928953 121.188953) (width 0.2) (layer "F.Cu") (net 6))
 (segment (start 148.954478 112.074062) (end 148.889713 112.10089) (width 0.2) (layer "F.Cu") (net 6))
 (segment (start 148.624531 112.119528) (end 148.276106 112.467953) (width 0.2) (layer "F.Cu") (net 6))
 (segment (start 149.015186 112.03901) (end 148.954478 112.074062) (width 0.2) (layer "F.Cu") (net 6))
 (segment (start 149.095971 111.971935) (end 149.0708 111.996333) (width 0.2) (layer "F.Cu") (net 6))
 (segment (start 151.918953 109.148953) (end 164.418953 109.148953) (width 0.2) (layer "F.Cu") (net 6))
 (segment (start 151.918953 109.148953) (end 149.095971 111.971935) (width 0.2) (layer "F.Cu") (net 6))
 (segment (start 149.0708 111.996333) (end 149.015186 112.03901) (width 0.2) (layer "F.Cu") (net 6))
 (arc (start 148.276106 112.467953) (mid 142.154339 113.685648) (end 136.964556 117.153351) (width 0.2) (layer "F.Cu") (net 6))
 (segment (start 148.12391 111.029488) (end 145.191866 111.029488) (width 0.2) (layer "F.Cu") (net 4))
 (segment (start 147.648837 110.508837) (end 148.168953 111.028953) (width 0.2) (layer "F.Cu") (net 4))
 (segment (start 148.168953 111.028953) (end 148.12391 111.029488) (width 0.2) (layer "F.Cu") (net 4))
 (arc (start 143.978953 101.648953) (mid 144.932725 106.443888) (end 147.648837 110.508837) (width 0.2) (layer "F.Cu") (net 4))
 (arc (start 145.191866 111.029488) (mid 138.555226 112.349598) (end 132.928953 116.108953) (width 0.2) (layer "F.Cu") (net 4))
 (segment (start 139.168953 108.432893) (end 139.168953 110.648953) (width 0.2) (layer "F.Cu") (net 23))
 (via (at 139.168953 110.648953) (size 0.6) (drill 0.3) (layers "F.Cu" "B.Cu") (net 23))
 (arc (start 136.358953 101.648953) (mid 138.438658 104.761451) (end 139.168953 108.432893) (width 0.2) (layer "F.Cu") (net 23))
 (segment (start 143.85 121.95) (end 148.168953 126.268953) (width 0.2) (layer "B.Cu") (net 23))
 (arc (start 139.168953 110.648953) (mid 140.385517 116.765036) (end 143.85 121.95) (width 0.2) (layer "B.Cu") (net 23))
 (segment (start 151.918953 114.148953) (end 164.418953 114.148953) (width 0.2) (layer "F.Cu") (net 31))
 (segment (start 129.418953 114.148953) (end 116.918953 114.148953) (width 0.2) (layer "F.Cu") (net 30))
 (via (at 130.593953 117.148953) (size 0.6) (drill 0.3) (layers "F.Cu" "B.Cu") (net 30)))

